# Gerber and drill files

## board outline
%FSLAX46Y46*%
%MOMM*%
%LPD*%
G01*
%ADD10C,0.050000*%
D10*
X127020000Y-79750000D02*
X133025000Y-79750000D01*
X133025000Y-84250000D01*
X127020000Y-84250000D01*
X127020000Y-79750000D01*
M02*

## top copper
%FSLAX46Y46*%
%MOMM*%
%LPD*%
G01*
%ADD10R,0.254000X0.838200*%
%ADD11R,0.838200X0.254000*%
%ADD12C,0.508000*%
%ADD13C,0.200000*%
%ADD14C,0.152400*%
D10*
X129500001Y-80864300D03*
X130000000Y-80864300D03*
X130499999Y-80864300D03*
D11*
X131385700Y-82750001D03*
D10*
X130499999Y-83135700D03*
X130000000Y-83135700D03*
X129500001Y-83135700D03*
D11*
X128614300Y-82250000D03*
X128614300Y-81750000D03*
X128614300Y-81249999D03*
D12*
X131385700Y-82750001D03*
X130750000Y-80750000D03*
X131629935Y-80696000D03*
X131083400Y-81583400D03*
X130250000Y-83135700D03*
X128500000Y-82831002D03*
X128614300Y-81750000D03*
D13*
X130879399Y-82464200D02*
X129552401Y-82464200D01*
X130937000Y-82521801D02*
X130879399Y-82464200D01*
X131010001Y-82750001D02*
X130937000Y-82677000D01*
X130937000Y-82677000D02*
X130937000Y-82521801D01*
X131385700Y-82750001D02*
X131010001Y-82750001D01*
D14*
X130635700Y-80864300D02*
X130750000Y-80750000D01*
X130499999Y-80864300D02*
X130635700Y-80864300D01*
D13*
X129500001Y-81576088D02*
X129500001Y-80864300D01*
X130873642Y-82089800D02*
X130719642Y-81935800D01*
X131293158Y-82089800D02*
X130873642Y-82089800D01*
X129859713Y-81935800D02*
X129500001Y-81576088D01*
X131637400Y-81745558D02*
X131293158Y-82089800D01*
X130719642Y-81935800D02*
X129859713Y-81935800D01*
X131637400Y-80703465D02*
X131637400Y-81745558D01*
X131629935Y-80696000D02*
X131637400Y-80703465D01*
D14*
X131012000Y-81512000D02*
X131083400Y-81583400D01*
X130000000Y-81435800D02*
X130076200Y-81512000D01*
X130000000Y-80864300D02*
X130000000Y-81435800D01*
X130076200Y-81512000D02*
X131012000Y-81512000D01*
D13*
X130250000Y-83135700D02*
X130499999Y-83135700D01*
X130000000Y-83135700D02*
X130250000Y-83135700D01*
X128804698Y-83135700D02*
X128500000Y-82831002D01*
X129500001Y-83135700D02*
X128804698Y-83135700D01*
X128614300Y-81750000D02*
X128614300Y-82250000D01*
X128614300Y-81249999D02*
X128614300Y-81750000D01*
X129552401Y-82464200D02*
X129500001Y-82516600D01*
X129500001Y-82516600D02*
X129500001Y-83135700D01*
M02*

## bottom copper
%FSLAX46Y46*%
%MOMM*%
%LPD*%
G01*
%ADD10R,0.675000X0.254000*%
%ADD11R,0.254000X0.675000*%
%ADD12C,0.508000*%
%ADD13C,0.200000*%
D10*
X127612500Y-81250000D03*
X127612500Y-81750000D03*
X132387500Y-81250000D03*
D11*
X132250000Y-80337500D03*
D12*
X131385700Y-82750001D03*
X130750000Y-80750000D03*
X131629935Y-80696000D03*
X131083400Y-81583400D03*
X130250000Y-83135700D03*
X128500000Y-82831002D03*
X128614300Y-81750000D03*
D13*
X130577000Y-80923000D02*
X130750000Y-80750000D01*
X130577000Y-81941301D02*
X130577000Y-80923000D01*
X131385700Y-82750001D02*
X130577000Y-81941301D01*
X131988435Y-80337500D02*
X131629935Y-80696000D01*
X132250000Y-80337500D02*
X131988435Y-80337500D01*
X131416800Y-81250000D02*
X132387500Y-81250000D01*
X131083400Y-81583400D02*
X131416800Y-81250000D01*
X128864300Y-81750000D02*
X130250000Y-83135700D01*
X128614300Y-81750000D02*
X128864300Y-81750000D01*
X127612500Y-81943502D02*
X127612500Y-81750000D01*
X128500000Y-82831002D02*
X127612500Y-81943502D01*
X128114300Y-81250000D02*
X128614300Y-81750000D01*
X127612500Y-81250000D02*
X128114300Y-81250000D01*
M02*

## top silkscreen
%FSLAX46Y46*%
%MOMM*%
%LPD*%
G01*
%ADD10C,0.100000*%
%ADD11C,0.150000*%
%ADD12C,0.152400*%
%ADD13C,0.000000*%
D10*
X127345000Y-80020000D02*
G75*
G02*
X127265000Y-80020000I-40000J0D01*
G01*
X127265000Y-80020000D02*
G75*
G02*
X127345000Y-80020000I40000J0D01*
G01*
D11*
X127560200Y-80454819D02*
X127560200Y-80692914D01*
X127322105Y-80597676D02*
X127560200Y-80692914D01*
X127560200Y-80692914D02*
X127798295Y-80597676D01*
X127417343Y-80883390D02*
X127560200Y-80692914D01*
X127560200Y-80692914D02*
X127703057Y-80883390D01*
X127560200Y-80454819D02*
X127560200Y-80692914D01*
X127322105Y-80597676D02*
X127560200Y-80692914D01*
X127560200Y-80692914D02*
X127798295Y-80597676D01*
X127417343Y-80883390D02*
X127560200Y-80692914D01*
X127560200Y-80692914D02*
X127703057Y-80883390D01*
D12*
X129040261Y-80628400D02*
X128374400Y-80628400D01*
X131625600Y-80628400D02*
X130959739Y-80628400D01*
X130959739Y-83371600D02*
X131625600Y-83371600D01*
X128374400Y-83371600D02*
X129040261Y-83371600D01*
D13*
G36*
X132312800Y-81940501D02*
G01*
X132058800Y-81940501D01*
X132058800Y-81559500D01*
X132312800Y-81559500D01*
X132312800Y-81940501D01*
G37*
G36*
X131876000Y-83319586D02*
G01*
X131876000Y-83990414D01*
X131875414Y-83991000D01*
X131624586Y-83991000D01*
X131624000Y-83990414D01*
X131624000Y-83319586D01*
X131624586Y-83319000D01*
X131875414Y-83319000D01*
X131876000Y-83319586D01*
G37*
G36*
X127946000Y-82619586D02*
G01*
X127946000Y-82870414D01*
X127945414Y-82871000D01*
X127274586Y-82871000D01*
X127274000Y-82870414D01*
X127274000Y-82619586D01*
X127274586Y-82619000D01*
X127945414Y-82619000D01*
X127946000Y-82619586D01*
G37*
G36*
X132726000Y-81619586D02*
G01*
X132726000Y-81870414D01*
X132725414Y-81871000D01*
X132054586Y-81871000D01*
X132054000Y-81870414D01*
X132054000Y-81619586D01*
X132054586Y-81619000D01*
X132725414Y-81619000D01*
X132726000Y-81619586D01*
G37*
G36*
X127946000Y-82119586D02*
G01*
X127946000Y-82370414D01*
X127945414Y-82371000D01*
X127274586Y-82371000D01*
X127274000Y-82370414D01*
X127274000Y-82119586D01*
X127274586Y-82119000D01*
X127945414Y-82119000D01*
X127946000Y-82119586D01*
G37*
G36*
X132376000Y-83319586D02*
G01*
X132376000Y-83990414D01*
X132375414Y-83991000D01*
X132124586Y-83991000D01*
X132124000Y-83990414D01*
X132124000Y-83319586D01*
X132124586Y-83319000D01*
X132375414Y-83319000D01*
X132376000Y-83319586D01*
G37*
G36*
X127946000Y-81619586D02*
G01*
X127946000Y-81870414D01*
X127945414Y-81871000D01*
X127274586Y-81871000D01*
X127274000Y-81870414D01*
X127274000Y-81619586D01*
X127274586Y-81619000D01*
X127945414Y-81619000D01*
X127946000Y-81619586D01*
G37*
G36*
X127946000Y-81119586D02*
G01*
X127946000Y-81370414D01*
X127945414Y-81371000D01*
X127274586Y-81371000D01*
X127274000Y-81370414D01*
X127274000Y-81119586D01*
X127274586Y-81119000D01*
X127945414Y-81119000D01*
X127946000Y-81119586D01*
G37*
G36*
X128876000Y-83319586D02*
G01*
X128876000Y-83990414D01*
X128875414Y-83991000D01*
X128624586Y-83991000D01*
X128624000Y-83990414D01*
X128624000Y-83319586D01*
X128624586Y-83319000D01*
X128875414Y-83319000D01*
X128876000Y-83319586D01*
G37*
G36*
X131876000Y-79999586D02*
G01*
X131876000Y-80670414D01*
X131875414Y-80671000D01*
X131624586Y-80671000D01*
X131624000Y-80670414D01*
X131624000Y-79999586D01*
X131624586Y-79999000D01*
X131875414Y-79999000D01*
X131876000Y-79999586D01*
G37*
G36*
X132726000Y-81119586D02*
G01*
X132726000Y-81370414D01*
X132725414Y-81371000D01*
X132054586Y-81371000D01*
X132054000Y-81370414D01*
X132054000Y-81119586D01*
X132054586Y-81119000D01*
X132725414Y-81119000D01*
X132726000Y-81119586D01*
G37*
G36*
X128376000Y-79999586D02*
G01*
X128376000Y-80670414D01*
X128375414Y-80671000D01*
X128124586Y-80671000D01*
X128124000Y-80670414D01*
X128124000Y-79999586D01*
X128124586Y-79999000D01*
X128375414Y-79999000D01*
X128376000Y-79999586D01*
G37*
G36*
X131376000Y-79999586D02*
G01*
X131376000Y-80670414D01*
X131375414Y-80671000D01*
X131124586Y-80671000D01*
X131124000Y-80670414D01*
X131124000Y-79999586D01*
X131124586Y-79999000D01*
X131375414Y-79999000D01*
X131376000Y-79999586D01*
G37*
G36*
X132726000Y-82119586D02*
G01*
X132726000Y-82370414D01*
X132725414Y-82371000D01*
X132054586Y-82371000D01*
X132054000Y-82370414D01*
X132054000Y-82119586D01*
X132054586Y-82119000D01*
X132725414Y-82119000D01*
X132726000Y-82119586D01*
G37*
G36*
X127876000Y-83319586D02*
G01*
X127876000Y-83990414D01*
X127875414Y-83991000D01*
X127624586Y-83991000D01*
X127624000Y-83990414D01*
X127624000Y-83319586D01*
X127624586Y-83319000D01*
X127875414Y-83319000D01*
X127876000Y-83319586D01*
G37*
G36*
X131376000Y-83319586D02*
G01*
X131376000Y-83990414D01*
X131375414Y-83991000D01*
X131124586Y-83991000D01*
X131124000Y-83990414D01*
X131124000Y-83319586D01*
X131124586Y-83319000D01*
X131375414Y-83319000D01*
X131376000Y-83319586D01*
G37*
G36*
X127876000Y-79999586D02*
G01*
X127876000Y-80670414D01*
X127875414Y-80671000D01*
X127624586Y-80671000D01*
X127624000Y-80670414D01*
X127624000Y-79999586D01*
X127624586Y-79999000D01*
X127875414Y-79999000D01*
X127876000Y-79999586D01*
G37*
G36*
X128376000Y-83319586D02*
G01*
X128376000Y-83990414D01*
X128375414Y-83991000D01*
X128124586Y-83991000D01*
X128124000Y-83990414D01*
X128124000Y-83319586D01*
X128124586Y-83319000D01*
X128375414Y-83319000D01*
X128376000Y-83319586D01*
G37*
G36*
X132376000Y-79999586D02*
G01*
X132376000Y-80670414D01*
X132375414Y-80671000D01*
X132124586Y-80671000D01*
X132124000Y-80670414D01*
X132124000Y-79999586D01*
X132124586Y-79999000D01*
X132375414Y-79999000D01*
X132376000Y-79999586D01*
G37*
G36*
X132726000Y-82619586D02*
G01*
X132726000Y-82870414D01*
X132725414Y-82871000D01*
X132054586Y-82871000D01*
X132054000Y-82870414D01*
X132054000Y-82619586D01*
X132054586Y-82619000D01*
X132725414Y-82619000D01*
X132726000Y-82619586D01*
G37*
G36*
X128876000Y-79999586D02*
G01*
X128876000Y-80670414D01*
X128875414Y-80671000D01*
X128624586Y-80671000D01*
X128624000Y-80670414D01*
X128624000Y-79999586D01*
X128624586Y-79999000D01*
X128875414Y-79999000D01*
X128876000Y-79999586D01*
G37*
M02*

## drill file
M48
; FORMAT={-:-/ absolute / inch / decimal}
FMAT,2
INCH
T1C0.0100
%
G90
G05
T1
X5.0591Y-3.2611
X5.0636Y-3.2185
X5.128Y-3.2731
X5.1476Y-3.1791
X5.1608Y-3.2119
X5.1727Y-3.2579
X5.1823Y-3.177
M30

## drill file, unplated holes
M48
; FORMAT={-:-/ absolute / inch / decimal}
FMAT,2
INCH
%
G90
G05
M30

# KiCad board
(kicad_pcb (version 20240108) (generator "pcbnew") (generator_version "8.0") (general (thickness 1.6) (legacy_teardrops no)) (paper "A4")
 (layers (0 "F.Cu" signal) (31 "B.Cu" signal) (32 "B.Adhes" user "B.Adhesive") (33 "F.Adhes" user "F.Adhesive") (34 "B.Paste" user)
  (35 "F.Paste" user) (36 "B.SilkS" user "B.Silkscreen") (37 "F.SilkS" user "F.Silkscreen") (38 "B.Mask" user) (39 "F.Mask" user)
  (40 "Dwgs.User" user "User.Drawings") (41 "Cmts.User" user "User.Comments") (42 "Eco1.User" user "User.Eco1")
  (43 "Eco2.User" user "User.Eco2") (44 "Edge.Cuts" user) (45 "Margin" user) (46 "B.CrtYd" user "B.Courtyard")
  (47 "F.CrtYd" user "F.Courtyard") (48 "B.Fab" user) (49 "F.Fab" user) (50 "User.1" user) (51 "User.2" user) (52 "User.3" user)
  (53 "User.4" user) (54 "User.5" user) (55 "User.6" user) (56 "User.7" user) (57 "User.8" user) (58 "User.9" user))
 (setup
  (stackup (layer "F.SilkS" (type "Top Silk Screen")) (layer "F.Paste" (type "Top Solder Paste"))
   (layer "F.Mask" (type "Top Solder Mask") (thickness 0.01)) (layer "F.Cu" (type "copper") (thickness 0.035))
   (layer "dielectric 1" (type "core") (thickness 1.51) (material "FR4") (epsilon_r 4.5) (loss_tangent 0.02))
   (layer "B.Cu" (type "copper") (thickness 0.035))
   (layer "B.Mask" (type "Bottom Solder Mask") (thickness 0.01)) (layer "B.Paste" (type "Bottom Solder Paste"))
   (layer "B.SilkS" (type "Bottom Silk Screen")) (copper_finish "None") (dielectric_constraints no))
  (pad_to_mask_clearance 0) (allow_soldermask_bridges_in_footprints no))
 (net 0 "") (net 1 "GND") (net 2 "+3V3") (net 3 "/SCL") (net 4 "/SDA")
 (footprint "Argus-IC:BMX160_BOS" (layer "F.Cu") (at 130 82)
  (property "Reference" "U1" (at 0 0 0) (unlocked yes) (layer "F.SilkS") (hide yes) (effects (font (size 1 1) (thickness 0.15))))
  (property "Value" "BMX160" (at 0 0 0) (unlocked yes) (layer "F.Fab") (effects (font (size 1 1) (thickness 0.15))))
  (fp_line (start -1.6256 1.3716) (end -0.959739 1.3716) (stroke (width 0.1524) (type solid)) (layer "F.SilkS"))
  (fp_line (start -0.959739 -1.3716) (end -1.6256 -1.3716) (stroke (width 0.1524) (type solid)) (layer "F.SilkS"))
  (fp_line (start 0.959739 1.3716) (end 1.6256 1.3716) (stroke (width 0.1524) (type solid)) (layer "F.SilkS"))
  (fp_line (start 1.6256 -1.3716) (end 0.959739 -1.3716) (stroke (width 0.1524) (type solid)) (layer "F.SilkS"))
  (fp_poly
   (pts (xy 2.3128 -0.4405) (xy 2.3128 -0.059499) (xy 2.0588 -0.059499) (xy 2.0588 -0.4405)) (stroke (width 0) (type solid)) (fill solid)
   (layer "F.SilkS"))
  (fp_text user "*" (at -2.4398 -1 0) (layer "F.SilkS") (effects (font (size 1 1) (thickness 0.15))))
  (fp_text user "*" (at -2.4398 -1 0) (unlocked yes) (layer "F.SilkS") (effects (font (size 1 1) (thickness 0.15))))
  (pad "1" smd rect (at -1.3857 -0.750001 90) (size 0.254 0.8382) (layers "F.Cu" "F.Paste" "F.Mask") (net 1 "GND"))
  (pad "2" smd rect (at -1.3857 -0.25 90) (size 0.254 0.8382) (layers "F.Cu" "F.Paste" "F.Mask") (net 1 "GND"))
  (pad "3" smd rect (at -1.3857 0.25 90) (size 0.254 0.8382) (layers "F.Cu" "F.Paste" "F.Mask") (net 1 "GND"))
  (pad "5" smd rect (at -0.499999 1.1357) (size 0.254 0.8382) (layers "F.Cu" "F.Paste" "F.Mask") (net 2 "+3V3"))
  (pad "6" smd rect (at 0 1.1357) (size 0.254 0.8382) (layers "F.Cu" "F.Paste" "F.Mask") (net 1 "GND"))
  (pad "7" smd rect (at 0.499999 1.1357) (size 0.254 0.8382) (layers "F.Cu" "F.Paste" "F.Mask") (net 1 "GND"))
  (pad "8" smd rect (at 1.3857 0.750001 90) (size 0.254 0.8382) (layers "F.Cu" "F.Paste" "F.Mask") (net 2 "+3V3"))
  (pad "12" smd rect (at 0.499999 -1.1357) (size 0.254 0.8382) (layers "F.Cu" "F.Paste" "F.Mask") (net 2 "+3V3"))
  (pad "13" smd rect (at 0 -1.1357) (size 0.254 0.8382) (layers "F.Cu" "F.Paste" "F.Mask") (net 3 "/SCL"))
  (pad "14" smd rect (at -0.499999 -1.1357) (size 0.254 0.8382) (layers "F.Cu" "F.Paste" "F.Mask") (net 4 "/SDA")))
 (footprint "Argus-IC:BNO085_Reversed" (layer "B.Cu") (at 130 82 180)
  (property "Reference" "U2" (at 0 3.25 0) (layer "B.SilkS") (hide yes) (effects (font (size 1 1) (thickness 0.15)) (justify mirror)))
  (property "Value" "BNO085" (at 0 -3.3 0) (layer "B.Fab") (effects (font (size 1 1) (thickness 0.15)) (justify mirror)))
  (pad "2" smd rect (at 2.3875 0.75 270) (size 0.254 0.675) (layers "B.Cu" "B.Paste" "B.Mask") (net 1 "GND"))
  (pad "3" smd rect (at 2.3875 0.25 270) (size 0.254 0.675) (layers "B.Cu" "B.Paste" "B.Mask") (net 2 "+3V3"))
  (pad "19" smd rect (at -2.3875 0.75 270) (size 0.254 0.675) (layers "B.Cu" "B.Paste" "B.Mask") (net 3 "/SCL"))
  (pad "20" smd rect (at -2.25 1.6625 180) (size 0.254 0.675) (layers "B.Cu" "B.Paste" "B.Mask") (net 4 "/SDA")))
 (gr_circle (center 127.305 80.02) (end 127.305 79.98) (stroke (width 0.1) (type default)) (fill none) (layer "F.SilkS"))
 (gr_rect (start 127.02 79.75) (end 133.025 84.25) (stroke (width 0.05) (type default)) (fill none) (layer "Edge.Cuts"))
 (segment (start 128.6143 81.75) (end 128.6143 82.25) (width 0.2) (layer "F.Cu") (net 1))
 (segment (start 130.25 83.1357) (end 130.499999 83.1357) (width 0.2) (layer "F.Cu") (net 1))
 (segment (start 128.6143 81.249999) (end 128.6143 81.75) (width 0.2) (layer "F.Cu") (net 1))
 (segment (start 130 83.1357) (end 130.25 83.1357) (width 0.2) (layer "F.Cu") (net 1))
 (via (at 128.6143 81.75) (size 0.508) (drill 0.254) (layers "F.Cu" "B.Cu") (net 1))
 (via (at 130.25 83.1357) (size 0.508) (drill 0.254) (layers "F.Cu" "B.Cu") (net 1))
 (segment (start 128.6143 81.75) (end 128.8643 81.75) (width 0.2) (layer "B.Cu") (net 1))
 (segment (start 128.8643 81.75) (end 130.25 83.1357) (width 0.2) (layer "B.Cu") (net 1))
 (segment (start 127.6125 81.25) (end 128.1143 81.25) (width 0.2) (layer "B.Cu") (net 1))
 (segment (start 128.1143 81.25) (end 128.6143 81.75) (width 0.2) (layer "B.Cu") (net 1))
 (segment (start 130.0762 81.512) (end 131.012 81.512) (width 0.1524) (layer "F.Cu") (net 3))
 (segment (start 131.012 81.512) (end 131.0834 81.5834) (width 0.1524) (layer "F.Cu") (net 3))
 (segment (start 130 81.4358) (end 130.0762 81.512) (width 0.1524) (layer "F.Cu") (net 3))
 (segment (start 130 80.8643) (end 130 81.4358) (width 0.1524) (layer "F.Cu") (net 3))
 (via (at 131.0834 81.5834) (size 0.508) (drill 0.254) (layers "F.Cu" "B.Cu") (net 3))
 (segment (start 131.4168 81.25) (end 132.3875 81.25) (width 0.2) (layer "B.Cu") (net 3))
 (segment (start 131.0834 81.5834) (end 131.4168 81.25) (width 0.2) (layer "B.Cu") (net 3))
 (segment (start 131.6374 80.703465) (end 131.6374 81.745558) (width 0.2) (layer "F.Cu") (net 4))
 (segment (start 131.629935 80.696) (end 131.6374 80.703465) (width 0.2) (layer "F.Cu") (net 4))
 (segment (start 130.873642 82.0898) (end 130.719642 81.9358) (width 0.2) (layer "F.Cu") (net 4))
 (segment (start 131.293158 82.0898) (end 130.873642 82.0898) (width 0.2) (layer "F.Cu") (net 4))
 (segment (start 130.719642 81.9358) (end 129.859713 81.9358) (width 0.2) (layer "F.Cu") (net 4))
 (segment (start 129.859713 81.9358) (end 129.500001 81.576088) (width 0.2) (layer "F.Cu") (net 4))
 (segment (start 131.6374 81.745558) (end 131.293158 82.0898) (width 0.2) (layer "F.Cu") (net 4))
 (segment (start 129.500001 81.576088) (end 129.500001 80.8643) (width 0.2) (layer "F.Cu") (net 4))
 (via (at 131.629935 80.696) (size 0.508) (drill 0.254) (layers "F.Cu" "B.Cu") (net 4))
 (segment (start 131.988435 80.3375) (end 131.629935 80.696) (width 0.2) (layer "B.Cu") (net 4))
 (segment (start 132.25 80.3375) (end 131.988435 80.3375) (width 0.2) (layer "B.Cu") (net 4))
 (segment (start 128.804698 83.1357) (end 128.5 82.831002) (width 0.2) (layer "F.Cu") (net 2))
 (segment (start 129.500001 82.5166) (end 129.500001 83.1357) (width 0.2) (layer "F.Cu") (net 2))
 (segment (start 130.937 82.521801) (end 130.879399 82.4642) (width 0.2) (layer "F.Cu") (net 2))
 (segment (start 130.937 82.677) (end 130.937 82.521801) (width 0.2) (layer "F.Cu") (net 2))
 (segment (start 129.500001 83.1357) (end 128.804698 83.1357) (width 0.2) (layer "F.Cu") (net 2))
 (segment (start 129.552401 82.4642) (end 129.500001 82.5166) (width 0.2) (layer "F.Cu") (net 2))
 (segment (start 131.010001 82.750001) (end 130.937 82.677) (width 0.2) (layer "F.Cu") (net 2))
 (segment (start 130.879399 82.4642) (end 129.552401 82.4642) (width 0.2) (layer "F.Cu") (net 2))
 (segment (start 130.6357 80.8643) (end 130.75 80.75) (width 0.1524) (layer "F.Cu") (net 2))
 (segment (start 131.3857 82.750001) (end 131.010001 82.750001) (width 0.2) (layer "F.Cu") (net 2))
 (segment (start 130.499999 80.8643) (end 130.6357 80.8643) (width 0.1524) (layer "F.Cu") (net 2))
 (via (at 130.75 80.75) (size 0.508) (drill 0.254) (layers "F.Cu" "B.Cu") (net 2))
 (via (at 131.3857 82.750001) (size 0.508) (drill 0.254) (layers "F.Cu" "B.Cu") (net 2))
 (via (at 128.5 82.831002) (size 0.508) (drill 0.254) (layers "F.Cu" "B.Cu") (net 2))
 (segment (start 130.577 81.941301) (end 130.577 80.923) (width 0.2) (layer "B.Cu") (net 2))
 (segment (start 131.3857 82.750001) (end 130.577 81.941301) (width 0.2) (layer "B.Cu") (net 2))
 (segment (start 127.6125 81.943502) (end 127.6125 81.75) (width 0.2) (layer "B.Cu") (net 2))
 (segment (start 128.5 82.831002) (end 127.6125 81.943502) (width 0.2) (layer "B.Cu") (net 2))
 (segment (start 130.577 80.923) (end 130.75 80.75) (width 0.2) (layer "B.Cu") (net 2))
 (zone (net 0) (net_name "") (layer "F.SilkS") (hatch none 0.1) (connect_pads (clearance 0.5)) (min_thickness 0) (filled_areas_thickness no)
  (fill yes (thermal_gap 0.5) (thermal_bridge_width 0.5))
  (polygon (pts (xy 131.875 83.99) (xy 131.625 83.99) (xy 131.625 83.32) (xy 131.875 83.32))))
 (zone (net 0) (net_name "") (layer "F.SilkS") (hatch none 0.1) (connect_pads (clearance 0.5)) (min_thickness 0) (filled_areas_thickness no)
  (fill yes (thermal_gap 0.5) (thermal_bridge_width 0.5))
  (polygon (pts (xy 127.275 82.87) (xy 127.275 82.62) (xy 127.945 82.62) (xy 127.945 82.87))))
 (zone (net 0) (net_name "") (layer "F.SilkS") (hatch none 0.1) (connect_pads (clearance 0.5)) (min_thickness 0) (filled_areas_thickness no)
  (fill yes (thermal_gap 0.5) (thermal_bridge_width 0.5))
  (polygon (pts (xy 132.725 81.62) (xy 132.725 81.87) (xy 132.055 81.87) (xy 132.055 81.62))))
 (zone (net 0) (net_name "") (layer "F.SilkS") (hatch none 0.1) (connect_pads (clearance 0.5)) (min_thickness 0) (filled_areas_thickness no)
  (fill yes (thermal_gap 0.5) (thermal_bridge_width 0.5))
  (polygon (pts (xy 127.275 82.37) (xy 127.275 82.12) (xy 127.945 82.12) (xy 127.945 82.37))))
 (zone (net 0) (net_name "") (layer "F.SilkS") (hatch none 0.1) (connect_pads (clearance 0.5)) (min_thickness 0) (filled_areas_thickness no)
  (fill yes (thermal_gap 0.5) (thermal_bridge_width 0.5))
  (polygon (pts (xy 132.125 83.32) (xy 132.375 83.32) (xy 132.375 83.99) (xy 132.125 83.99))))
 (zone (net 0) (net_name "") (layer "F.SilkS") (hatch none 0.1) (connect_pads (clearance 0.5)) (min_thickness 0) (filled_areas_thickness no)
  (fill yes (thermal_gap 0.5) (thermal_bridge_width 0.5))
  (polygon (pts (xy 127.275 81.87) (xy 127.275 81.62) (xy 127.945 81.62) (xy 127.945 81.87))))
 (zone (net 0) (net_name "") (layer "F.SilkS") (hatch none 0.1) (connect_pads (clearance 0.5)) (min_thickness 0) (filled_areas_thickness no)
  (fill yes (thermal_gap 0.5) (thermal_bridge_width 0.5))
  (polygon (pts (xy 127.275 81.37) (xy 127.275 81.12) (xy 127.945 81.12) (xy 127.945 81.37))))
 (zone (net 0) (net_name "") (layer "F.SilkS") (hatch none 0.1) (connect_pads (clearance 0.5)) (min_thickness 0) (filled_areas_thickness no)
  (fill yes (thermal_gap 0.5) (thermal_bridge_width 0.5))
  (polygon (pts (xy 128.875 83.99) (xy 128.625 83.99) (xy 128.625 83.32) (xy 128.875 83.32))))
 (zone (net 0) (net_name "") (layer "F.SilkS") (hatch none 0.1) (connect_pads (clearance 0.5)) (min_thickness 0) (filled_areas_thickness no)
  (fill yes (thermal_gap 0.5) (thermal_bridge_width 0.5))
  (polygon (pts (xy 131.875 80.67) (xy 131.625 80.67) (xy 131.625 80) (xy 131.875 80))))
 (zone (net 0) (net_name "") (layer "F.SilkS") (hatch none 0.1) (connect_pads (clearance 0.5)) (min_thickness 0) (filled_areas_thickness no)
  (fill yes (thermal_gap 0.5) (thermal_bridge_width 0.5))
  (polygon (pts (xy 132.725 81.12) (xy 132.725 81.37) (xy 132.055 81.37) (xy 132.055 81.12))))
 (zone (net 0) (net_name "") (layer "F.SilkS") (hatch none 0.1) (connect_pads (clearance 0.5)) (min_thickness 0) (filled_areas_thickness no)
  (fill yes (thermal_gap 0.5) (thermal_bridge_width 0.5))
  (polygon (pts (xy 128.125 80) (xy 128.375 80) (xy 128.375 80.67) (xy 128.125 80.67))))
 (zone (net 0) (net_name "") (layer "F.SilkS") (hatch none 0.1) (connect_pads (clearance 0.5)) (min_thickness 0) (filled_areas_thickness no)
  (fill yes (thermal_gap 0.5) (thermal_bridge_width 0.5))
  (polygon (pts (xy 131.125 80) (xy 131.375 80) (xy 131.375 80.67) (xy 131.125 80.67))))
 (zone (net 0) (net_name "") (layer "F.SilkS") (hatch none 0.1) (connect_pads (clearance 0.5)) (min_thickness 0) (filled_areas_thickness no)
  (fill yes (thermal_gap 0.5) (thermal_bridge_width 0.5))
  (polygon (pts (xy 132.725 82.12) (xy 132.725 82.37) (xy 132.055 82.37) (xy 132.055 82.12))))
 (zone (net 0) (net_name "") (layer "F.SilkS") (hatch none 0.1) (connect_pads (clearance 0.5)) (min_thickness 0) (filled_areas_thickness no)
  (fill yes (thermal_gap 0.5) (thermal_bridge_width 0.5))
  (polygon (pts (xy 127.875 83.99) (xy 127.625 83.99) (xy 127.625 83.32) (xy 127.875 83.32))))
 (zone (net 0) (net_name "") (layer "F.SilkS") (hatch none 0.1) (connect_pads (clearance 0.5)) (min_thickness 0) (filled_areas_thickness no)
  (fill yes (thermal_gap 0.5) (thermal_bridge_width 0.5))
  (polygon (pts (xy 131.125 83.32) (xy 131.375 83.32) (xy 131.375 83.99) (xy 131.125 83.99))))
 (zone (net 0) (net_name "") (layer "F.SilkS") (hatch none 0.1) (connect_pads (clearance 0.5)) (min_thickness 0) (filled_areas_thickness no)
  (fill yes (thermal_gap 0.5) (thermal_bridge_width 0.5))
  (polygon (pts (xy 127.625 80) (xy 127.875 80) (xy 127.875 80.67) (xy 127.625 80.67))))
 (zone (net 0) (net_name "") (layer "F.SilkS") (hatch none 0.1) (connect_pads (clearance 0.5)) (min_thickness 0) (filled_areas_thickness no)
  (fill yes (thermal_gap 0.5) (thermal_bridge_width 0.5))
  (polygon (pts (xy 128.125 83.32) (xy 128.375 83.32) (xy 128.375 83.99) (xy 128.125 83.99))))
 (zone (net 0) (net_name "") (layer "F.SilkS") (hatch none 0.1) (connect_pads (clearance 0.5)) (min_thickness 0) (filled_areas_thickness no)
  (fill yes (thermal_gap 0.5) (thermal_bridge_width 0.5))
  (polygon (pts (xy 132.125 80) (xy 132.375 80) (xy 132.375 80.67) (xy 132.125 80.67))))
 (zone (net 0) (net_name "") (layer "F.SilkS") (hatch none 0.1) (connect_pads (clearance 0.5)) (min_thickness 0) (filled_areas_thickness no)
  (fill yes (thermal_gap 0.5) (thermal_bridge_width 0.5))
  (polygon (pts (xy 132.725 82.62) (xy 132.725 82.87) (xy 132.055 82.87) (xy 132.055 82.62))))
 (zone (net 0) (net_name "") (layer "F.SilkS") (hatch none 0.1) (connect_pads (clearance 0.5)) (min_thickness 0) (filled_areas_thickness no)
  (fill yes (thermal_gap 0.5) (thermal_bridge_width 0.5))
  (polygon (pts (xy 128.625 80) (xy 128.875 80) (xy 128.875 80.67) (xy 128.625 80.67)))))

